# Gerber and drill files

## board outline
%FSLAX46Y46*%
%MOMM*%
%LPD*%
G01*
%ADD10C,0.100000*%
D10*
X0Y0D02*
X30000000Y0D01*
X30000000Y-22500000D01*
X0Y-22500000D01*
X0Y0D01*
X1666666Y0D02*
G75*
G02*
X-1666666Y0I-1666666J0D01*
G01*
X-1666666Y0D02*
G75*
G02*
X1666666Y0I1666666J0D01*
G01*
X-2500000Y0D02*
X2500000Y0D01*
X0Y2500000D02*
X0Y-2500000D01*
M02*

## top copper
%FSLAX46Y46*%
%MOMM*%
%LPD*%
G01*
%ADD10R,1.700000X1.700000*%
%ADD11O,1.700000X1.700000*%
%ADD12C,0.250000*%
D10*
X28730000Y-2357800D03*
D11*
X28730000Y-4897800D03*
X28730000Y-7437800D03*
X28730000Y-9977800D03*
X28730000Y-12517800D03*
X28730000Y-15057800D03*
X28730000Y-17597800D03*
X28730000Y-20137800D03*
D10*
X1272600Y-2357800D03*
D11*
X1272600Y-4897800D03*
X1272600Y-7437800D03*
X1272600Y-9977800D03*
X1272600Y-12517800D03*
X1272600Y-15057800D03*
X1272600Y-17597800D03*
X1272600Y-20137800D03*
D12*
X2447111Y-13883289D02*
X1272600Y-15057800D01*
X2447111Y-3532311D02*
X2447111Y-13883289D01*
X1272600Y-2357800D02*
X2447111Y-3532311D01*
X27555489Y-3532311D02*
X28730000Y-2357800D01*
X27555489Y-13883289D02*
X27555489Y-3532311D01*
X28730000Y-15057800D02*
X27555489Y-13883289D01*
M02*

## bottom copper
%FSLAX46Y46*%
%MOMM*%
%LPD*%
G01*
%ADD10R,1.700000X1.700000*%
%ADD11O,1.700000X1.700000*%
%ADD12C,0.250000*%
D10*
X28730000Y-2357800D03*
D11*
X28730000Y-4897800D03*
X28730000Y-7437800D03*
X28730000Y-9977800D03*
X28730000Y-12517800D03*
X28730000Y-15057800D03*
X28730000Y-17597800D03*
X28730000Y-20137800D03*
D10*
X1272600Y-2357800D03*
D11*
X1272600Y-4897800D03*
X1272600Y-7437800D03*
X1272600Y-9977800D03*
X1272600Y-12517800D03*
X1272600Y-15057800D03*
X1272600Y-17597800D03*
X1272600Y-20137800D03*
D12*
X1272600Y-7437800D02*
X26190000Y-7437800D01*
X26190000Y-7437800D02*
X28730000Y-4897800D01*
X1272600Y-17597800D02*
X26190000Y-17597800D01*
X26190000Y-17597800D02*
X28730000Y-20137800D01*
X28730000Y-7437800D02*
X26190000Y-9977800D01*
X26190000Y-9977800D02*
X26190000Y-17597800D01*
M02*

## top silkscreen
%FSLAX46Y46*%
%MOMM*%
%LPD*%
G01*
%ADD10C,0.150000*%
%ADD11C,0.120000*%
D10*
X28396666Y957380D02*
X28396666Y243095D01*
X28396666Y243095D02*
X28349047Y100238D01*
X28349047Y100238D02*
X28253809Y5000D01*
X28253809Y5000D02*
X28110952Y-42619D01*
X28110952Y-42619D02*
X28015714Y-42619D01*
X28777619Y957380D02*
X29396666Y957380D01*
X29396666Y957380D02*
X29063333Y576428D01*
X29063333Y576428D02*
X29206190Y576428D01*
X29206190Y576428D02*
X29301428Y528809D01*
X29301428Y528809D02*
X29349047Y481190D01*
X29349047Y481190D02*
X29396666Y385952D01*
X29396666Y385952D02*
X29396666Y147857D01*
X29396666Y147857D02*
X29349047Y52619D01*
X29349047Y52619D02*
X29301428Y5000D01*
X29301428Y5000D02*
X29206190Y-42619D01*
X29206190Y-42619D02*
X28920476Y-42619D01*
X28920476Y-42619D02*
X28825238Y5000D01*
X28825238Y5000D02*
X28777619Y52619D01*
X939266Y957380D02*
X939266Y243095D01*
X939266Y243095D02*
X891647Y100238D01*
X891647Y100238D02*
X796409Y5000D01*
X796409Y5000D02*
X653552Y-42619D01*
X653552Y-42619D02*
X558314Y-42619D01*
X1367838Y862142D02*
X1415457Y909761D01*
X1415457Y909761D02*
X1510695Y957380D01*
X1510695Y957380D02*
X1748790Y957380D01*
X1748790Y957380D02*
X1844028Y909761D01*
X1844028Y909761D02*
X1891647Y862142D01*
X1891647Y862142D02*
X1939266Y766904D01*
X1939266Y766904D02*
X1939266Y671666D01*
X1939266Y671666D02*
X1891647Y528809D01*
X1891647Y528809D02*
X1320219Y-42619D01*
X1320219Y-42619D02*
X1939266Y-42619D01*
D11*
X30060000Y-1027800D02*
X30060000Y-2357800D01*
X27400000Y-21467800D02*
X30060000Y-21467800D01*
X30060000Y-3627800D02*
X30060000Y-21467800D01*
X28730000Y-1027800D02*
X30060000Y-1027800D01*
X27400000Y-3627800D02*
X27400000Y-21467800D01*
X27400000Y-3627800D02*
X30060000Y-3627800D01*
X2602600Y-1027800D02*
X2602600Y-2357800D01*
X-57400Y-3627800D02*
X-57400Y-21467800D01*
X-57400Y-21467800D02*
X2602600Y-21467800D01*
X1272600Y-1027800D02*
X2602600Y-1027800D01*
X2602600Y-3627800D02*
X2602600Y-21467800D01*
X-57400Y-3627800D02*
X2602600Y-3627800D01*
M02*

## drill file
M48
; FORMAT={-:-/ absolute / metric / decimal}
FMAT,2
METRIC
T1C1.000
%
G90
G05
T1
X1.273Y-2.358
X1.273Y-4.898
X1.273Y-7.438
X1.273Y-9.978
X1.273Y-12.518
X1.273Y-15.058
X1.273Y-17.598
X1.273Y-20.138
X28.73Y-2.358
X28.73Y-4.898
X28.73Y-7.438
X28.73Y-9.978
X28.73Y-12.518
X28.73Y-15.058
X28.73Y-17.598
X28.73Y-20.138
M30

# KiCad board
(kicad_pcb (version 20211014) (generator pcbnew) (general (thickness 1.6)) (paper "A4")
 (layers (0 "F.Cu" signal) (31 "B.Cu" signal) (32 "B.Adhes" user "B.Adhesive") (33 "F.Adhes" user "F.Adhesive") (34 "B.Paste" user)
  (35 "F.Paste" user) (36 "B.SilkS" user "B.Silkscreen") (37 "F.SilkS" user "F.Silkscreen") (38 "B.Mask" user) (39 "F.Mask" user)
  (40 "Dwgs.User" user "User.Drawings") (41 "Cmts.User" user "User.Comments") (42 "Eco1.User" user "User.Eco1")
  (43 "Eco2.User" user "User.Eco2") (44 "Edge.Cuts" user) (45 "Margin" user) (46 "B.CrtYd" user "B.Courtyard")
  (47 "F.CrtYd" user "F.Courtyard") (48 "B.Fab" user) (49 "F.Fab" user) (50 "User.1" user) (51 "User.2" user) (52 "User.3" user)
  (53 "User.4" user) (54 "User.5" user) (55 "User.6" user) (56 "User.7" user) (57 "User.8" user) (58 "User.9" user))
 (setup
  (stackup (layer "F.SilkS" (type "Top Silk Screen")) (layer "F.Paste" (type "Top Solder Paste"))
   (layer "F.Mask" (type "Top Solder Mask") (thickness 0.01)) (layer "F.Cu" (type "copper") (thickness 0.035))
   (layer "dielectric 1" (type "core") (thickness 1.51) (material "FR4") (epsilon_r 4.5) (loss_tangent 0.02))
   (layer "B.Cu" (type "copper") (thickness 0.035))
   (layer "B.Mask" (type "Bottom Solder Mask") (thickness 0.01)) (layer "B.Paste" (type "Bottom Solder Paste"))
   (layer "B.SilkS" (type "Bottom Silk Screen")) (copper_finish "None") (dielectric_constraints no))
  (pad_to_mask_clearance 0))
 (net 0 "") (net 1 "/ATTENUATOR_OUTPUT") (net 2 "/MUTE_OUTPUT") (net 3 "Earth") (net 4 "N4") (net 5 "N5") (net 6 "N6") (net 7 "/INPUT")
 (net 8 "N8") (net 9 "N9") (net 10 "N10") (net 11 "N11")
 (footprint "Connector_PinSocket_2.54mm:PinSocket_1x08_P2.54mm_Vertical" (layer "F.Cu") (at 28.73 2.3578)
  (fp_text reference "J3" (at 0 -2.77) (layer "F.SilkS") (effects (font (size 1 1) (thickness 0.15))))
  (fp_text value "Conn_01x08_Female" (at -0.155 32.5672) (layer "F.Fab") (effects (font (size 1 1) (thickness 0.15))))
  (fp_line (start 1.33 -1.33) (end 1.33 0) (layer "F.SilkS") (width 0.12))
  (fp_line (start -1.33 19.11) (end 1.33 19.11) (layer "F.SilkS") (width 0.12))
  (fp_line (start 1.33 1.27) (end 1.33 19.11) (layer "F.SilkS") (width 0.12))
  (fp_line (start 0 -1.33) (end 1.33 -1.33) (layer "F.SilkS") (width 0.12))
  (fp_line (start -1.33 1.27) (end -1.33 19.11) (layer "F.SilkS") (width 0.12))
  (fp_line (start -1.33 1.27) (end 1.33 1.27) (layer "F.SilkS") (width 0.12))
  (pad "1" thru_hole rect (at 0 0) (size 1.7 1.7) (drill 1) (layers *.Cu *.Mask) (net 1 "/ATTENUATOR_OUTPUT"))
  (pad "2" thru_hole oval (at 0 2.54) (size 1.7 1.7) (drill 1) (layers *.Cu *.Mask) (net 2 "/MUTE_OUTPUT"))
  (pad "3" thru_hole oval (at 0 5.08) (size 1.7 1.7) (drill 1) (layers *.Cu *.Mask) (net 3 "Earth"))
  (pad "4" thru_hole oval (at 0 7.62) (size 1.7 1.7) (drill 1) (layers *.Cu *.Mask) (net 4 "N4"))
  (pad "5" thru_hole oval (at 0 10.16) (size 1.7 1.7) (drill 1) (layers *.Cu *.Mask) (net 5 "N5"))
  (pad "6" thru_hole oval (at 0 12.7) (size 1.7 1.7) (drill 1) (layers *.Cu *.Mask) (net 1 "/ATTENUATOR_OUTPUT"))
  (pad "7" thru_hole oval (at 0 15.24) (size 1.7 1.7) (drill 1) (layers *.Cu *.Mask) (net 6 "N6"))
  (pad "8" thru_hole oval (at 0 17.78) (size 1.7 1.7) (drill 1) (layers *.Cu *.Mask) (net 3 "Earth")))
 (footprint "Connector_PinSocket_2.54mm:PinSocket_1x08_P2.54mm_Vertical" (layer "F.Cu") (at 1.2726 2.3578)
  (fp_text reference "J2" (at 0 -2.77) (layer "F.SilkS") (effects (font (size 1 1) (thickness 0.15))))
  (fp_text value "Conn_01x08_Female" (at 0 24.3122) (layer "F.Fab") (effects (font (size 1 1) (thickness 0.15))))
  (fp_line (start 1.33 -1.33) (end 1.33 0) (layer "F.SilkS") (width 0.12))
  (fp_line (start -1.33 1.27) (end -1.33 19.11) (layer "F.SilkS") (width 0.12))
  (fp_line (start -1.33 19.11) (end 1.33 19.11) (layer "F.SilkS") (width 0.12))
  (fp_line (start 0 -1.33) (end 1.33 -1.33) (layer "F.SilkS") (width 0.12))
  (fp_line (start 1.33 1.27) (end 1.33 19.11) (layer "F.SilkS") (width 0.12))
  (fp_line (start -1.33 1.27) (end 1.33 1.27) (layer "F.SilkS") (width 0.12))
  (pad "1" thru_hole rect (at 0 0) (size 1.7 1.7) (drill 1) (layers *.Cu *.Mask) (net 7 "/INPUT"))
  (pad "2" thru_hole oval (at 0 2.54) (size 1.7 1.7) (drill 1) (layers *.Cu *.Mask) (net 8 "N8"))
  (pad "3" thru_hole oval (at 0 5.08) (size 1.7 1.7) (drill 1) (layers *.Cu *.Mask) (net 2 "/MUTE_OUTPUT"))
  (pad "4" thru_hole oval (at 0 7.62) (size 1.7 1.7) (drill 1) (layers *.Cu *.Mask) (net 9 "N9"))
  (pad "5" thru_hole oval (at 0 10.16) (size 1.7 1.7) (drill 1) (layers *.Cu *.Mask) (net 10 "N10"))
  (pad "6" thru_hole oval (at 0 12.7) (size 1.7 1.7) (drill 1) (layers *.Cu *.Mask) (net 7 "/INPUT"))
  (pad "7" thru_hole oval (at 0 15.24) (size 1.7 1.7) (drill 1) (layers *.Cu *.Mask) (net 3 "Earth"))
  (pad "8" thru_hole oval (at 0 17.78) (size 1.7 1.7) (drill 1) (layers *.Cu *.Mask) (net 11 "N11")))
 (gr_rect (start 0 0) (end 30 22.5) (layer "Edge.Cuts") (width 0.1) (fill none))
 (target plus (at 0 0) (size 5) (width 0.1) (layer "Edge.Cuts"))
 (segment (start 2.447111 13.883289) (end 1.2726 15.0578) (width 0.25) (layer "F.Cu") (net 7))
 (segment (start 2.447111 3.532311) (end 2.447111 13.883289) (width 0.25) (layer "F.Cu") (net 7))
 (segment (start 1.2726 2.3578) (end 2.447111 3.532311) (width 0.25) (layer "F.Cu") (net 7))
 (segment (start 1.2726 7.4378) (end 26.19 7.4378) (width 0.25) (layer "B.Cu") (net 2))
 (segment (start 26.19 7.4378) (end 28.73 4.8978) (width 0.25) (layer "B.Cu") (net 2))
 (segment (start 1.2726 17.5978) (end 26.19 17.5978) (width 0.25) (layer "B.Cu") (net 3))
 (segment (start 26.19 17.5978) (end 28.73 20.1378) (width 0.25) (layer "B.Cu") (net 3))
 (segment (start 28.73 7.4378) (end 26.19 9.9778) (width 0.25) (layer "B.Cu") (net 3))
 (segment (start 26.19 9.9778) (end 26.19 17.5978) (width 0.25) (layer "B.Cu") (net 3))
 (segment (start 27.555489 3.532311) (end 28.73 2.3578) (width 0.25) (layer "F.Cu") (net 1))
 (segment (start 27.555489 13.883289) (end 27.555489 3.532311) (width 0.25) (layer "F.Cu") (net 1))
 (segment (start 28.73 15.0578) (end 27.555489 13.883289) (width 0.25) (layer "F.Cu") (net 1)))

